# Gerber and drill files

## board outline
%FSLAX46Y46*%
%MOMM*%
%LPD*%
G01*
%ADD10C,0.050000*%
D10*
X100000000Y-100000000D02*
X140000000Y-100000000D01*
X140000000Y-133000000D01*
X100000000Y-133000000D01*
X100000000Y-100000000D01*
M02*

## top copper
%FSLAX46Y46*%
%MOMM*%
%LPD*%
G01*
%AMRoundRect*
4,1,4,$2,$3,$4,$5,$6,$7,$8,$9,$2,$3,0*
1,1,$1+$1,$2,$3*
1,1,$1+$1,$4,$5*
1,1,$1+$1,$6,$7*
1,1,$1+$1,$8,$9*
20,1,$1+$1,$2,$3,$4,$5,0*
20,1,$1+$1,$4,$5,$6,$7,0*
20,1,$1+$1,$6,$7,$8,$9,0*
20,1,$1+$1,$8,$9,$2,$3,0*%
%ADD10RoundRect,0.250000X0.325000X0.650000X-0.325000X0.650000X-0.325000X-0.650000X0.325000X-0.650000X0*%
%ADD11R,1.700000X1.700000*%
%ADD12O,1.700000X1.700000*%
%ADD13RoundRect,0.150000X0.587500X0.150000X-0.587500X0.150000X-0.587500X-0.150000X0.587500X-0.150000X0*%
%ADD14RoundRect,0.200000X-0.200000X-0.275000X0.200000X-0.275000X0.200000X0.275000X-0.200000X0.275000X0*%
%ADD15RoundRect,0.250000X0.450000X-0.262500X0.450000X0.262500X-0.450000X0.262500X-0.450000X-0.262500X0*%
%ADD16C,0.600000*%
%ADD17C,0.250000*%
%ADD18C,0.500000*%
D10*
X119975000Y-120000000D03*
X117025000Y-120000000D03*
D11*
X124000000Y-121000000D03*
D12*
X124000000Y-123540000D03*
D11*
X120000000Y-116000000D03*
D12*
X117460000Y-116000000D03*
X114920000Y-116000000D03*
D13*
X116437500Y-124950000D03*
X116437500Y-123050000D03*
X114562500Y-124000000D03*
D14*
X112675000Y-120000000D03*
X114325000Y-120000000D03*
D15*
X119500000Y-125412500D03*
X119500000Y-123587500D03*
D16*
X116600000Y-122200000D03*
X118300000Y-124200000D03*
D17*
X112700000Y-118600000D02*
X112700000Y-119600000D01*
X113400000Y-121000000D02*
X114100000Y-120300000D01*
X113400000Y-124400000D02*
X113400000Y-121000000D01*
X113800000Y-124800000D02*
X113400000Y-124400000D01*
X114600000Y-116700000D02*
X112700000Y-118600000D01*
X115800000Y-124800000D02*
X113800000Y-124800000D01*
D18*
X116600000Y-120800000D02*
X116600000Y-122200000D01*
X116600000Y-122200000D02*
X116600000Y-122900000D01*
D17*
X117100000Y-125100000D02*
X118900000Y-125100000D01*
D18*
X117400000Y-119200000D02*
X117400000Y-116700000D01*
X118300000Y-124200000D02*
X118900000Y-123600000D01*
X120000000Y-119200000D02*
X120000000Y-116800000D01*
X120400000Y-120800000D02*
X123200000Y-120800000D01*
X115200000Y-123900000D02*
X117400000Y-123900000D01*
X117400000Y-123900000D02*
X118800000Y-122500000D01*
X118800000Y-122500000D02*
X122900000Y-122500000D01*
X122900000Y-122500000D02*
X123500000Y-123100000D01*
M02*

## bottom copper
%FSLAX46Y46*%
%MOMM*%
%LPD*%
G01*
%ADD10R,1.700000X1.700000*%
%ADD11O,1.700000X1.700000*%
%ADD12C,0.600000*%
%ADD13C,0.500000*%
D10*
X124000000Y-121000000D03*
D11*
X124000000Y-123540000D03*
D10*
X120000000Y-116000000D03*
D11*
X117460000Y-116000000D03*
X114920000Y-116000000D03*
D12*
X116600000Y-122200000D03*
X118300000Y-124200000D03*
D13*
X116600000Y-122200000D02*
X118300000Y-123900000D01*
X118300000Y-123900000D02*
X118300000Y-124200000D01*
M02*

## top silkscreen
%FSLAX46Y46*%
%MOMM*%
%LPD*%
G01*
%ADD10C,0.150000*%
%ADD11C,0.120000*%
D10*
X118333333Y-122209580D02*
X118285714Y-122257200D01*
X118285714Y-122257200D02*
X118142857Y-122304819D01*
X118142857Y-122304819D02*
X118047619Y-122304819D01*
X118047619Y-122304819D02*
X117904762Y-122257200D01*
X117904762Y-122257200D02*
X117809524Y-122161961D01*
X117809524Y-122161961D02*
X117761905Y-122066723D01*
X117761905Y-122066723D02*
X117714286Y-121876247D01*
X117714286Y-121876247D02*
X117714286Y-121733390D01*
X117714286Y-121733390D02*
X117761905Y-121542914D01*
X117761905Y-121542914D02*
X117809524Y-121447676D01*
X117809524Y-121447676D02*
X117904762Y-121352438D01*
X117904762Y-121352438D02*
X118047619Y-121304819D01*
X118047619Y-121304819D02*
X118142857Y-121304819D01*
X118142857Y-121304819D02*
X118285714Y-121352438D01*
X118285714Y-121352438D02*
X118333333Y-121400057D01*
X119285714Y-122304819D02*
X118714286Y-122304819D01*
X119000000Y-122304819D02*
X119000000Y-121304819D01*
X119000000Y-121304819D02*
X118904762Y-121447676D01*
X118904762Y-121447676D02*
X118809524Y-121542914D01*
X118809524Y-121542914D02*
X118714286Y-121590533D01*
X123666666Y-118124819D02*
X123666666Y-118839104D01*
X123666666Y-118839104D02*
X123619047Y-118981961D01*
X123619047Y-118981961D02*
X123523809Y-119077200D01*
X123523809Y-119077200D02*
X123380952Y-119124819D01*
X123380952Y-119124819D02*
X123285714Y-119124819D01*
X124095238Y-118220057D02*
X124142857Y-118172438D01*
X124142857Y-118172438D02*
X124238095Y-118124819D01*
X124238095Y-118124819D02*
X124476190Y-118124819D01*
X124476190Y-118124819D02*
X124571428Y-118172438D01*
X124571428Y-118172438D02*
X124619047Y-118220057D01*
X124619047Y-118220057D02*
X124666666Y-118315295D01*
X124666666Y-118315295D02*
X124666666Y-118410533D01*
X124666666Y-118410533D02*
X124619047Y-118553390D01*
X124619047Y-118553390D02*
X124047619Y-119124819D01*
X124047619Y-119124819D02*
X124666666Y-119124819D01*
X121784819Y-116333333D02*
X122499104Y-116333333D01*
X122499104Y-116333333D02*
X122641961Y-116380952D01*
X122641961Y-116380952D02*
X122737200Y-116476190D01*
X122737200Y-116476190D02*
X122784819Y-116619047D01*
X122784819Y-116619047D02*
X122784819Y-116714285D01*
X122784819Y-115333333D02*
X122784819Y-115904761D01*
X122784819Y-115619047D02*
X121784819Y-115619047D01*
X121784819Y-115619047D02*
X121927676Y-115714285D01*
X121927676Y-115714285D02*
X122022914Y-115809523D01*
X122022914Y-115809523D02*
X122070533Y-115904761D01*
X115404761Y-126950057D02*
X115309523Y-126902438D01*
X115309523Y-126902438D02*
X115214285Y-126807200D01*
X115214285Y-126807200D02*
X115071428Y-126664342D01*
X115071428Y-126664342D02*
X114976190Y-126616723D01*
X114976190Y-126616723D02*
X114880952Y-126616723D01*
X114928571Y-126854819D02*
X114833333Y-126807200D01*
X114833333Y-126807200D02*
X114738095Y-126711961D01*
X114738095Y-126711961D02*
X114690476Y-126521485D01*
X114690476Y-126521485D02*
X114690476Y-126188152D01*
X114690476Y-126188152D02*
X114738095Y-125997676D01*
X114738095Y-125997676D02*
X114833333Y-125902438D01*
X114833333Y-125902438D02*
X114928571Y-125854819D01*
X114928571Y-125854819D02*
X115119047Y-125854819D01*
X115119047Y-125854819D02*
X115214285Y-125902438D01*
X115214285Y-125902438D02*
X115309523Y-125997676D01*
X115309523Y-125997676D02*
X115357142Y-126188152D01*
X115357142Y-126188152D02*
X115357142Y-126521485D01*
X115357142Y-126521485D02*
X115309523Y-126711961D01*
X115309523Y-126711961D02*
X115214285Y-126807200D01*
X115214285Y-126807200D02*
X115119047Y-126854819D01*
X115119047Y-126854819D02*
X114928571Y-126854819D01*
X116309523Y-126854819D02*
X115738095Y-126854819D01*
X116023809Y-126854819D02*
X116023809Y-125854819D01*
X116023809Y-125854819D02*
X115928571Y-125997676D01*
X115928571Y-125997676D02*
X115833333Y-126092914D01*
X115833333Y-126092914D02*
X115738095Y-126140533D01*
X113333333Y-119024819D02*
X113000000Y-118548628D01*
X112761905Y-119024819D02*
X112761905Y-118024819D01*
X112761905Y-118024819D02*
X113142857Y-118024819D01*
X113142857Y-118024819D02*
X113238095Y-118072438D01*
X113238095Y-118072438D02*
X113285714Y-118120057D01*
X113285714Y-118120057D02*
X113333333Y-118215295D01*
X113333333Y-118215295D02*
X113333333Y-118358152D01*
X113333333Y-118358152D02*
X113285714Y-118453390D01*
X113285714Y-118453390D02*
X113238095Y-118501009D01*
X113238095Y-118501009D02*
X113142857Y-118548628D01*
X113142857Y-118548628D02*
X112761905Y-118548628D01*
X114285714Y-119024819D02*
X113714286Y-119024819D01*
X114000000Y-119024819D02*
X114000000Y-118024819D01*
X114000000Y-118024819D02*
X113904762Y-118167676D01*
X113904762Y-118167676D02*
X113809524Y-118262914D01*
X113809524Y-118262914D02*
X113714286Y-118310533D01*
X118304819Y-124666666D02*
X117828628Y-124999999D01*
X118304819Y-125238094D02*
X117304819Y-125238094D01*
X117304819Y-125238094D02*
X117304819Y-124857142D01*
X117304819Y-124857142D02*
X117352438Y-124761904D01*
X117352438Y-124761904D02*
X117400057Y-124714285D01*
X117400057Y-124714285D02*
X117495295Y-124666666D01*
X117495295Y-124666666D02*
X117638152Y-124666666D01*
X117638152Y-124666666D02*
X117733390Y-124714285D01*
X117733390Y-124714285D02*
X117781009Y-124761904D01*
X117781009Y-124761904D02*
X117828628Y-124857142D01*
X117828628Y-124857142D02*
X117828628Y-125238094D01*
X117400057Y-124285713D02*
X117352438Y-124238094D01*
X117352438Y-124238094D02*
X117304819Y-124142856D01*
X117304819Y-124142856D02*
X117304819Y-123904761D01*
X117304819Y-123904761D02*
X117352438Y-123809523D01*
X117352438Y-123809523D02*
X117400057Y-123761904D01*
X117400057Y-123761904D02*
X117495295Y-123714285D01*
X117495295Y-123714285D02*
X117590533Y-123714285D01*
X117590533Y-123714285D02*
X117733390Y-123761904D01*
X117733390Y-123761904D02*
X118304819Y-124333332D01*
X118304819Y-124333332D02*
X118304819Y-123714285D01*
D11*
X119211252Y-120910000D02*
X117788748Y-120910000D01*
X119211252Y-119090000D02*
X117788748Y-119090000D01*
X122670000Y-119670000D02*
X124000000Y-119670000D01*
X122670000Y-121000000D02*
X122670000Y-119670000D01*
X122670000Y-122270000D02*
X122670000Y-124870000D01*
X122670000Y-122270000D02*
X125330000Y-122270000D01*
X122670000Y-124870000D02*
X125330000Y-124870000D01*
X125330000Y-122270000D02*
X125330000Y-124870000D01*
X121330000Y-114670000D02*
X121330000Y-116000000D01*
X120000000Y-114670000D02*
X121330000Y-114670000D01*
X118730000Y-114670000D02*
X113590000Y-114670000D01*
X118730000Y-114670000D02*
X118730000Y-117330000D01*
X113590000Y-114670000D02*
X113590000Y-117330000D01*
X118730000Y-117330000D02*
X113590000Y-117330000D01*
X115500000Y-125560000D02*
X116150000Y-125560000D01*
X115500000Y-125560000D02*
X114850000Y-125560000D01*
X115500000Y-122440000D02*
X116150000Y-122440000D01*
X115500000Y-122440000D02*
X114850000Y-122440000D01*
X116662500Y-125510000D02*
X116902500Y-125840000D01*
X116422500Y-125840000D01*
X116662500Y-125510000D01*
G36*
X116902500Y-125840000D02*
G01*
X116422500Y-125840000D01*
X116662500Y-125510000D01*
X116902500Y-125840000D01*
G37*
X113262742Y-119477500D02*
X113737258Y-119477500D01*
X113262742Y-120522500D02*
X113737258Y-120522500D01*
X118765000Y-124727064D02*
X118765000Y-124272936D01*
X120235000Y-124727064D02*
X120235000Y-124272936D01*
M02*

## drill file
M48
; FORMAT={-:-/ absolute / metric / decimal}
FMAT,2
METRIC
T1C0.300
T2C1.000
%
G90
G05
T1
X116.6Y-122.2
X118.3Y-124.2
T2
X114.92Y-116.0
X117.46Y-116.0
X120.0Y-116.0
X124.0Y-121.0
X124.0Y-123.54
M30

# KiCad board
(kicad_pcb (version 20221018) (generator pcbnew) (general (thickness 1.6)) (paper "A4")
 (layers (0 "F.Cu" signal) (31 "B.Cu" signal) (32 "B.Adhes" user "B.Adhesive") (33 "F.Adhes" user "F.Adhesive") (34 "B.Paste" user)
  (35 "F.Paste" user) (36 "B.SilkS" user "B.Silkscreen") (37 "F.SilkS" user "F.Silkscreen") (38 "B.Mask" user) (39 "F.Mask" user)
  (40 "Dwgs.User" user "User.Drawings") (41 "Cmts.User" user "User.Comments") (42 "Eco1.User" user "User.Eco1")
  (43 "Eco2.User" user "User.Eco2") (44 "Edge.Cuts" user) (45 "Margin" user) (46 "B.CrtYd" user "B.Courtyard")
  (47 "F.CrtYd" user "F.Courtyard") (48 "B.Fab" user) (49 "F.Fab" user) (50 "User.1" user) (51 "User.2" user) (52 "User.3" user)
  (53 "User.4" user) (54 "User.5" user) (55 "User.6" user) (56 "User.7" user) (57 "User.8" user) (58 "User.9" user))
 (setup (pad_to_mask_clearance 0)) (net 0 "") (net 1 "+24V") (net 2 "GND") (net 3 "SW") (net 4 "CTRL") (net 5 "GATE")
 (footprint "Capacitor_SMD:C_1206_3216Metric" (layer "F.Cu") (at 118.5 120 180)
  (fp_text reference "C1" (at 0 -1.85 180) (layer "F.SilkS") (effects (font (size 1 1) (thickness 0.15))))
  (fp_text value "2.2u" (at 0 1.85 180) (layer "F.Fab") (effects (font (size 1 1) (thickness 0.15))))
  (fp_line (start -0.711252 -0.91) (end 0.711252 -0.91) (stroke (width 0.12) (type solid)) (layer "F.SilkS"))
  (fp_line (start -0.711252 0.91) (end 0.711252 0.91) (stroke (width 0.12) (type solid)) (layer "F.SilkS"))
  (pad "1" smd roundrect (at -1.475 0 180) (size 1.15 1.8) (layers "F.Cu" "F.Paste" "F.Mask") (roundrect_rratio 0.217391) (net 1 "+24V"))
  (pad "2" smd roundrect (at 1.475 0 180) (size 1.15 1.8) (layers "F.Cu" "F.Paste" "F.Mask") (roundrect_rratio 0.217391) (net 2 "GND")))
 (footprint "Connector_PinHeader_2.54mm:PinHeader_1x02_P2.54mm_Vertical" (layer "F.Cu") (at 124 121)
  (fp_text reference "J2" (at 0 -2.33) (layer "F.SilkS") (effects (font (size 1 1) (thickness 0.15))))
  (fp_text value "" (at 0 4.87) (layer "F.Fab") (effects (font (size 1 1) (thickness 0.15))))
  (fp_line (start -1.33 -1.33) (end 0 -1.33) (stroke (width 0.12) (type solid)) (layer "F.SilkS"))
  (fp_line (start -1.33 0) (end -1.33 -1.33) (stroke (width 0.12) (type solid)) (layer "F.SilkS"))
  (fp_line (start -1.33 1.27) (end -1.33 3.87) (stroke (width 0.12) (type solid)) (layer "F.SilkS"))
  (fp_line (start -1.33 1.27) (end 1.33 1.27) (stroke (width 0.12) (type solid)) (layer "F.SilkS"))
  (fp_line (start -1.33 3.87) (end 1.33 3.87) (stroke (width 0.12) (type solid)) (layer "F.SilkS"))
  (fp_line (start 1.33 1.27) (end 1.33 3.87) (stroke (width 0.12) (type solid)) (layer "F.SilkS"))
  (pad "1" thru_hole rect (at 0 0) (size 1.7 1.7) (drill 1) (layers "*.Cu" "*.Mask") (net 1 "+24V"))
  (pad "2" thru_hole oval (at 0 2.54) (size 1.7 1.7) (drill 1) (layers "*.Cu" "*.Mask") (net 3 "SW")))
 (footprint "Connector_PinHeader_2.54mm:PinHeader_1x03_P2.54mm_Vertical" (layer "F.Cu") (at 120 116 -90)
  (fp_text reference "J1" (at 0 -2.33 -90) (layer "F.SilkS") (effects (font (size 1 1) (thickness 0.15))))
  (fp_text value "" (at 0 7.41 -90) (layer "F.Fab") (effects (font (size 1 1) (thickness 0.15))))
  (fp_line (start -1.33 -1.33) (end 0 -1.33) (stroke (width 0.12) (type solid)) (layer "F.SilkS"))
  (fp_line (start -1.33 0) (end -1.33 -1.33) (stroke (width 0.12) (type solid)) (layer "F.SilkS"))
  (fp_line (start -1.33 1.27) (end -1.33 6.41) (stroke (width 0.12) (type solid)) (layer "F.SilkS"))
  (fp_line (start -1.33 1.27) (end 1.33 1.27) (stroke (width 0.12) (type solid)) (layer "F.SilkS"))
  (fp_line (start -1.33 6.41) (end 1.33 6.41) (stroke (width 0.12) (type solid)) (layer "F.SilkS"))
  (fp_line (start 1.33 1.27) (end 1.33 6.41) (stroke (width 0.12) (type solid)) (layer "F.SilkS"))
  (pad "1" thru_hole rect (at 0 0 270) (size 1.7 1.7) (drill 1) (layers "*.Cu" "*.Mask") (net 1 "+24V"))
  (pad "2" thru_hole oval (at 0 2.54 270) (size 1.7 1.7) (drill 1) (layers "*.Cu" "*.Mask") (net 2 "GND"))
  (pad "3" thru_hole oval (at 0 5.08 270) (size 1.7 1.7) (drill 1) (layers "*.Cu" "*.Mask") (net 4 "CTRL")))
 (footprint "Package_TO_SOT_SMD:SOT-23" (layer "F.Cu") (at 115.5 124 180)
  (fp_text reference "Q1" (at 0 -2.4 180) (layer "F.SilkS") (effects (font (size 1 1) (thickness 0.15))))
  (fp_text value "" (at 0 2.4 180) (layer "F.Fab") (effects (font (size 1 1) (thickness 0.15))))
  (fp_line (start 0 -1.56) (end -0.65 -1.56) (stroke (width 0.12) (type solid)) (layer "F.SilkS"))
  (fp_line (start 0 -1.56) (end 0.65 -1.56) (stroke (width 0.12) (type solid)) (layer "F.SilkS"))
  (fp_line (start 0 1.56) (end -0.65 1.56) (stroke (width 0.12) (type solid)) (layer "F.SilkS"))
  (fp_line (start 0 1.56) (end 0.65 1.56) (stroke (width 0.12) (type solid)) (layer "F.SilkS"))
  (fp_poly
   (pts (xy -1.1625 -1.51) (xy -1.4025 -1.84) (xy -0.9225 -1.84) (xy -1.1625 -1.51)) (stroke (width 0.12) (type solid)) (fill solid)
   (layer "F.SilkS"))
  (pad "1" smd roundrect (at -0.9375 -0.95 180) (size 1.475 0.6) (layers "F.Cu" "F.Paste" "F.Mask") (roundrect_rratio 0.25) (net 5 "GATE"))
  (pad "2" smd roundrect (at -0.9375 0.95 180) (size 1.475 0.6) (layers "F.Cu" "F.Paste" "F.Mask") (roundrect_rratio 0.25) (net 2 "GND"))
  (pad "3" smd roundrect (at 0.9375 0 180) (size 1.475 0.6) (layers "F.Cu" "F.Paste" "F.Mask") (roundrect_rratio 0.25) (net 3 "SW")))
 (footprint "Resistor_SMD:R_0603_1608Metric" (layer "F.Cu") (at 113.5 120)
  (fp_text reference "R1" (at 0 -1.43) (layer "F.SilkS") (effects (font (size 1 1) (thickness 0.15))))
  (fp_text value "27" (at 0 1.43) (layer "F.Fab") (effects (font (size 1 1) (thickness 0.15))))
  (fp_line (start -0.237258 -0.5225) (end 0.237258 -0.5225) (stroke (width 0.12) (type solid)) (layer "F.SilkS"))
  (fp_line (start -0.237258 0.5225) (end 0.237258 0.5225) (stroke (width 0.12) (type solid)) (layer "F.SilkS"))
  (pad "1" smd roundrect (at -0.825 0) (size 0.8 0.95) (layers "F.Cu" "F.Paste" "F.Mask") (roundrect_rratio 0.25) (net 4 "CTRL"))
  (pad "2" smd roundrect (at 0.825 0) (size 0.8 0.95) (layers "F.Cu" "F.Paste" "F.Mask") (roundrect_rratio 0.25) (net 5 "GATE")))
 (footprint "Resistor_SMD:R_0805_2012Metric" (layer "F.Cu") (at 119.5 124.5 90)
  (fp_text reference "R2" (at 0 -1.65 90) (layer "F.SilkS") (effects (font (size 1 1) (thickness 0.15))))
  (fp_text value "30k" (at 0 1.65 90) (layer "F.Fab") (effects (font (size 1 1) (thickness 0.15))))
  (fp_line (start -0.227064 -0.735) (end 0.227064 -0.735) (stroke (width 0.12) (type solid)) (layer "F.SilkS"))
  (fp_line (start -0.227064 0.735) (end 0.227064 0.735) (stroke (width 0.12) (type solid)) (layer "F.SilkS"))
  (pad "1" smd roundrect (at -0.9125 0 90) (size 1.025 1.4) (layers "F.Cu" "F.Paste" "F.Mask") (roundrect_rratio 0.243902) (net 5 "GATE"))
  (pad "2" smd roundrect (at 0.9125 0 90) (size 1.025 1.4) (layers "F.Cu" "F.Paste" "F.Mask") (roundrect_rratio 0.243902) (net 2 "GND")))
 (gr_rect (start 100 100) (end 140 133) (stroke (width 0.05) (type default)) (fill none) (layer "Edge.Cuts"))
 (segment (start 112.7 118.6) (end 112.7 119.6) (width 0.25) (layer "F.Cu") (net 4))
 (segment (start 113.4 121) (end 114.1 120.3) (width 0.25) (layer "F.Cu") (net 5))
 (segment (start 113.4 124.4) (end 113.4 121) (width 0.25) (layer "F.Cu") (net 5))
 (segment (start 113.8 124.8) (end 113.4 124.4) (width 0.25) (layer "F.Cu") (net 5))
 (segment (start 114.6 116.7) (end 112.7 118.6) (width 0.25) (layer "F.Cu") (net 4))
 (segment (start 115.8 124.8) (end 113.8 124.8) (width 0.25) (layer "F.Cu") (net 5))
 (segment (start 116.6 120.8) (end 116.6 122.2) (width 0.5) (layer "F.Cu") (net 2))
 (segment (start 116.6 122.2) (end 116.6 122.9) (width 0.5) (layer "F.Cu") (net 2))
 (segment (start 117.1 125.1) (end 118.9 125.1) (width 0.25) (layer "F.Cu") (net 5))
 (segment (start 117.4 119.2) (end 117.4 116.7) (width 0.5) (layer "F.Cu") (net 2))
 (segment (start 118.3 124.2) (end 118.9 123.6) (width 0.5) (layer "F.Cu") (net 2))
 (segment (start 120 119.2) (end 120 116.8) (width 0.5) (layer "F.Cu") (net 1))
 (segment (start 120.4 120.8) (end 123.2 120.8) (width 0.5) (layer "F.Cu") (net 1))
 (via (at 116.6 122.2) (size 0.6) (drill 0.3) (layers "F.Cu" "B.Cu") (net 2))
 (via (at 118.3 124.2) (size 0.6) (drill 0.3) (layers "F.Cu" "B.Cu") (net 2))
 (segment (start 115.2 123.9) (end 117.4 123.9) (width 0.5) (layer "F.Cu") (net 3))
 (segment (start 116.6 122.2) (end 118.3 123.9) (width 0.5) (layer "B.Cu") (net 2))
 (segment (start 117.4 123.9) (end 118.8 122.5) (width 0.5) (layer "F.Cu") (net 3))
 (segment (start 118.3 123.9) (end 118.3 124.2) (width 0.5) (layer "B.Cu") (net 2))
 (segment (start 118.8 122.5) (end 122.9 122.5) (width 0.5) (layer "F.Cu") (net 3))
 (segment (start 122.9 122.5) (end 123.5 123.1) (width 0.5) (layer "F.Cu") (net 3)))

